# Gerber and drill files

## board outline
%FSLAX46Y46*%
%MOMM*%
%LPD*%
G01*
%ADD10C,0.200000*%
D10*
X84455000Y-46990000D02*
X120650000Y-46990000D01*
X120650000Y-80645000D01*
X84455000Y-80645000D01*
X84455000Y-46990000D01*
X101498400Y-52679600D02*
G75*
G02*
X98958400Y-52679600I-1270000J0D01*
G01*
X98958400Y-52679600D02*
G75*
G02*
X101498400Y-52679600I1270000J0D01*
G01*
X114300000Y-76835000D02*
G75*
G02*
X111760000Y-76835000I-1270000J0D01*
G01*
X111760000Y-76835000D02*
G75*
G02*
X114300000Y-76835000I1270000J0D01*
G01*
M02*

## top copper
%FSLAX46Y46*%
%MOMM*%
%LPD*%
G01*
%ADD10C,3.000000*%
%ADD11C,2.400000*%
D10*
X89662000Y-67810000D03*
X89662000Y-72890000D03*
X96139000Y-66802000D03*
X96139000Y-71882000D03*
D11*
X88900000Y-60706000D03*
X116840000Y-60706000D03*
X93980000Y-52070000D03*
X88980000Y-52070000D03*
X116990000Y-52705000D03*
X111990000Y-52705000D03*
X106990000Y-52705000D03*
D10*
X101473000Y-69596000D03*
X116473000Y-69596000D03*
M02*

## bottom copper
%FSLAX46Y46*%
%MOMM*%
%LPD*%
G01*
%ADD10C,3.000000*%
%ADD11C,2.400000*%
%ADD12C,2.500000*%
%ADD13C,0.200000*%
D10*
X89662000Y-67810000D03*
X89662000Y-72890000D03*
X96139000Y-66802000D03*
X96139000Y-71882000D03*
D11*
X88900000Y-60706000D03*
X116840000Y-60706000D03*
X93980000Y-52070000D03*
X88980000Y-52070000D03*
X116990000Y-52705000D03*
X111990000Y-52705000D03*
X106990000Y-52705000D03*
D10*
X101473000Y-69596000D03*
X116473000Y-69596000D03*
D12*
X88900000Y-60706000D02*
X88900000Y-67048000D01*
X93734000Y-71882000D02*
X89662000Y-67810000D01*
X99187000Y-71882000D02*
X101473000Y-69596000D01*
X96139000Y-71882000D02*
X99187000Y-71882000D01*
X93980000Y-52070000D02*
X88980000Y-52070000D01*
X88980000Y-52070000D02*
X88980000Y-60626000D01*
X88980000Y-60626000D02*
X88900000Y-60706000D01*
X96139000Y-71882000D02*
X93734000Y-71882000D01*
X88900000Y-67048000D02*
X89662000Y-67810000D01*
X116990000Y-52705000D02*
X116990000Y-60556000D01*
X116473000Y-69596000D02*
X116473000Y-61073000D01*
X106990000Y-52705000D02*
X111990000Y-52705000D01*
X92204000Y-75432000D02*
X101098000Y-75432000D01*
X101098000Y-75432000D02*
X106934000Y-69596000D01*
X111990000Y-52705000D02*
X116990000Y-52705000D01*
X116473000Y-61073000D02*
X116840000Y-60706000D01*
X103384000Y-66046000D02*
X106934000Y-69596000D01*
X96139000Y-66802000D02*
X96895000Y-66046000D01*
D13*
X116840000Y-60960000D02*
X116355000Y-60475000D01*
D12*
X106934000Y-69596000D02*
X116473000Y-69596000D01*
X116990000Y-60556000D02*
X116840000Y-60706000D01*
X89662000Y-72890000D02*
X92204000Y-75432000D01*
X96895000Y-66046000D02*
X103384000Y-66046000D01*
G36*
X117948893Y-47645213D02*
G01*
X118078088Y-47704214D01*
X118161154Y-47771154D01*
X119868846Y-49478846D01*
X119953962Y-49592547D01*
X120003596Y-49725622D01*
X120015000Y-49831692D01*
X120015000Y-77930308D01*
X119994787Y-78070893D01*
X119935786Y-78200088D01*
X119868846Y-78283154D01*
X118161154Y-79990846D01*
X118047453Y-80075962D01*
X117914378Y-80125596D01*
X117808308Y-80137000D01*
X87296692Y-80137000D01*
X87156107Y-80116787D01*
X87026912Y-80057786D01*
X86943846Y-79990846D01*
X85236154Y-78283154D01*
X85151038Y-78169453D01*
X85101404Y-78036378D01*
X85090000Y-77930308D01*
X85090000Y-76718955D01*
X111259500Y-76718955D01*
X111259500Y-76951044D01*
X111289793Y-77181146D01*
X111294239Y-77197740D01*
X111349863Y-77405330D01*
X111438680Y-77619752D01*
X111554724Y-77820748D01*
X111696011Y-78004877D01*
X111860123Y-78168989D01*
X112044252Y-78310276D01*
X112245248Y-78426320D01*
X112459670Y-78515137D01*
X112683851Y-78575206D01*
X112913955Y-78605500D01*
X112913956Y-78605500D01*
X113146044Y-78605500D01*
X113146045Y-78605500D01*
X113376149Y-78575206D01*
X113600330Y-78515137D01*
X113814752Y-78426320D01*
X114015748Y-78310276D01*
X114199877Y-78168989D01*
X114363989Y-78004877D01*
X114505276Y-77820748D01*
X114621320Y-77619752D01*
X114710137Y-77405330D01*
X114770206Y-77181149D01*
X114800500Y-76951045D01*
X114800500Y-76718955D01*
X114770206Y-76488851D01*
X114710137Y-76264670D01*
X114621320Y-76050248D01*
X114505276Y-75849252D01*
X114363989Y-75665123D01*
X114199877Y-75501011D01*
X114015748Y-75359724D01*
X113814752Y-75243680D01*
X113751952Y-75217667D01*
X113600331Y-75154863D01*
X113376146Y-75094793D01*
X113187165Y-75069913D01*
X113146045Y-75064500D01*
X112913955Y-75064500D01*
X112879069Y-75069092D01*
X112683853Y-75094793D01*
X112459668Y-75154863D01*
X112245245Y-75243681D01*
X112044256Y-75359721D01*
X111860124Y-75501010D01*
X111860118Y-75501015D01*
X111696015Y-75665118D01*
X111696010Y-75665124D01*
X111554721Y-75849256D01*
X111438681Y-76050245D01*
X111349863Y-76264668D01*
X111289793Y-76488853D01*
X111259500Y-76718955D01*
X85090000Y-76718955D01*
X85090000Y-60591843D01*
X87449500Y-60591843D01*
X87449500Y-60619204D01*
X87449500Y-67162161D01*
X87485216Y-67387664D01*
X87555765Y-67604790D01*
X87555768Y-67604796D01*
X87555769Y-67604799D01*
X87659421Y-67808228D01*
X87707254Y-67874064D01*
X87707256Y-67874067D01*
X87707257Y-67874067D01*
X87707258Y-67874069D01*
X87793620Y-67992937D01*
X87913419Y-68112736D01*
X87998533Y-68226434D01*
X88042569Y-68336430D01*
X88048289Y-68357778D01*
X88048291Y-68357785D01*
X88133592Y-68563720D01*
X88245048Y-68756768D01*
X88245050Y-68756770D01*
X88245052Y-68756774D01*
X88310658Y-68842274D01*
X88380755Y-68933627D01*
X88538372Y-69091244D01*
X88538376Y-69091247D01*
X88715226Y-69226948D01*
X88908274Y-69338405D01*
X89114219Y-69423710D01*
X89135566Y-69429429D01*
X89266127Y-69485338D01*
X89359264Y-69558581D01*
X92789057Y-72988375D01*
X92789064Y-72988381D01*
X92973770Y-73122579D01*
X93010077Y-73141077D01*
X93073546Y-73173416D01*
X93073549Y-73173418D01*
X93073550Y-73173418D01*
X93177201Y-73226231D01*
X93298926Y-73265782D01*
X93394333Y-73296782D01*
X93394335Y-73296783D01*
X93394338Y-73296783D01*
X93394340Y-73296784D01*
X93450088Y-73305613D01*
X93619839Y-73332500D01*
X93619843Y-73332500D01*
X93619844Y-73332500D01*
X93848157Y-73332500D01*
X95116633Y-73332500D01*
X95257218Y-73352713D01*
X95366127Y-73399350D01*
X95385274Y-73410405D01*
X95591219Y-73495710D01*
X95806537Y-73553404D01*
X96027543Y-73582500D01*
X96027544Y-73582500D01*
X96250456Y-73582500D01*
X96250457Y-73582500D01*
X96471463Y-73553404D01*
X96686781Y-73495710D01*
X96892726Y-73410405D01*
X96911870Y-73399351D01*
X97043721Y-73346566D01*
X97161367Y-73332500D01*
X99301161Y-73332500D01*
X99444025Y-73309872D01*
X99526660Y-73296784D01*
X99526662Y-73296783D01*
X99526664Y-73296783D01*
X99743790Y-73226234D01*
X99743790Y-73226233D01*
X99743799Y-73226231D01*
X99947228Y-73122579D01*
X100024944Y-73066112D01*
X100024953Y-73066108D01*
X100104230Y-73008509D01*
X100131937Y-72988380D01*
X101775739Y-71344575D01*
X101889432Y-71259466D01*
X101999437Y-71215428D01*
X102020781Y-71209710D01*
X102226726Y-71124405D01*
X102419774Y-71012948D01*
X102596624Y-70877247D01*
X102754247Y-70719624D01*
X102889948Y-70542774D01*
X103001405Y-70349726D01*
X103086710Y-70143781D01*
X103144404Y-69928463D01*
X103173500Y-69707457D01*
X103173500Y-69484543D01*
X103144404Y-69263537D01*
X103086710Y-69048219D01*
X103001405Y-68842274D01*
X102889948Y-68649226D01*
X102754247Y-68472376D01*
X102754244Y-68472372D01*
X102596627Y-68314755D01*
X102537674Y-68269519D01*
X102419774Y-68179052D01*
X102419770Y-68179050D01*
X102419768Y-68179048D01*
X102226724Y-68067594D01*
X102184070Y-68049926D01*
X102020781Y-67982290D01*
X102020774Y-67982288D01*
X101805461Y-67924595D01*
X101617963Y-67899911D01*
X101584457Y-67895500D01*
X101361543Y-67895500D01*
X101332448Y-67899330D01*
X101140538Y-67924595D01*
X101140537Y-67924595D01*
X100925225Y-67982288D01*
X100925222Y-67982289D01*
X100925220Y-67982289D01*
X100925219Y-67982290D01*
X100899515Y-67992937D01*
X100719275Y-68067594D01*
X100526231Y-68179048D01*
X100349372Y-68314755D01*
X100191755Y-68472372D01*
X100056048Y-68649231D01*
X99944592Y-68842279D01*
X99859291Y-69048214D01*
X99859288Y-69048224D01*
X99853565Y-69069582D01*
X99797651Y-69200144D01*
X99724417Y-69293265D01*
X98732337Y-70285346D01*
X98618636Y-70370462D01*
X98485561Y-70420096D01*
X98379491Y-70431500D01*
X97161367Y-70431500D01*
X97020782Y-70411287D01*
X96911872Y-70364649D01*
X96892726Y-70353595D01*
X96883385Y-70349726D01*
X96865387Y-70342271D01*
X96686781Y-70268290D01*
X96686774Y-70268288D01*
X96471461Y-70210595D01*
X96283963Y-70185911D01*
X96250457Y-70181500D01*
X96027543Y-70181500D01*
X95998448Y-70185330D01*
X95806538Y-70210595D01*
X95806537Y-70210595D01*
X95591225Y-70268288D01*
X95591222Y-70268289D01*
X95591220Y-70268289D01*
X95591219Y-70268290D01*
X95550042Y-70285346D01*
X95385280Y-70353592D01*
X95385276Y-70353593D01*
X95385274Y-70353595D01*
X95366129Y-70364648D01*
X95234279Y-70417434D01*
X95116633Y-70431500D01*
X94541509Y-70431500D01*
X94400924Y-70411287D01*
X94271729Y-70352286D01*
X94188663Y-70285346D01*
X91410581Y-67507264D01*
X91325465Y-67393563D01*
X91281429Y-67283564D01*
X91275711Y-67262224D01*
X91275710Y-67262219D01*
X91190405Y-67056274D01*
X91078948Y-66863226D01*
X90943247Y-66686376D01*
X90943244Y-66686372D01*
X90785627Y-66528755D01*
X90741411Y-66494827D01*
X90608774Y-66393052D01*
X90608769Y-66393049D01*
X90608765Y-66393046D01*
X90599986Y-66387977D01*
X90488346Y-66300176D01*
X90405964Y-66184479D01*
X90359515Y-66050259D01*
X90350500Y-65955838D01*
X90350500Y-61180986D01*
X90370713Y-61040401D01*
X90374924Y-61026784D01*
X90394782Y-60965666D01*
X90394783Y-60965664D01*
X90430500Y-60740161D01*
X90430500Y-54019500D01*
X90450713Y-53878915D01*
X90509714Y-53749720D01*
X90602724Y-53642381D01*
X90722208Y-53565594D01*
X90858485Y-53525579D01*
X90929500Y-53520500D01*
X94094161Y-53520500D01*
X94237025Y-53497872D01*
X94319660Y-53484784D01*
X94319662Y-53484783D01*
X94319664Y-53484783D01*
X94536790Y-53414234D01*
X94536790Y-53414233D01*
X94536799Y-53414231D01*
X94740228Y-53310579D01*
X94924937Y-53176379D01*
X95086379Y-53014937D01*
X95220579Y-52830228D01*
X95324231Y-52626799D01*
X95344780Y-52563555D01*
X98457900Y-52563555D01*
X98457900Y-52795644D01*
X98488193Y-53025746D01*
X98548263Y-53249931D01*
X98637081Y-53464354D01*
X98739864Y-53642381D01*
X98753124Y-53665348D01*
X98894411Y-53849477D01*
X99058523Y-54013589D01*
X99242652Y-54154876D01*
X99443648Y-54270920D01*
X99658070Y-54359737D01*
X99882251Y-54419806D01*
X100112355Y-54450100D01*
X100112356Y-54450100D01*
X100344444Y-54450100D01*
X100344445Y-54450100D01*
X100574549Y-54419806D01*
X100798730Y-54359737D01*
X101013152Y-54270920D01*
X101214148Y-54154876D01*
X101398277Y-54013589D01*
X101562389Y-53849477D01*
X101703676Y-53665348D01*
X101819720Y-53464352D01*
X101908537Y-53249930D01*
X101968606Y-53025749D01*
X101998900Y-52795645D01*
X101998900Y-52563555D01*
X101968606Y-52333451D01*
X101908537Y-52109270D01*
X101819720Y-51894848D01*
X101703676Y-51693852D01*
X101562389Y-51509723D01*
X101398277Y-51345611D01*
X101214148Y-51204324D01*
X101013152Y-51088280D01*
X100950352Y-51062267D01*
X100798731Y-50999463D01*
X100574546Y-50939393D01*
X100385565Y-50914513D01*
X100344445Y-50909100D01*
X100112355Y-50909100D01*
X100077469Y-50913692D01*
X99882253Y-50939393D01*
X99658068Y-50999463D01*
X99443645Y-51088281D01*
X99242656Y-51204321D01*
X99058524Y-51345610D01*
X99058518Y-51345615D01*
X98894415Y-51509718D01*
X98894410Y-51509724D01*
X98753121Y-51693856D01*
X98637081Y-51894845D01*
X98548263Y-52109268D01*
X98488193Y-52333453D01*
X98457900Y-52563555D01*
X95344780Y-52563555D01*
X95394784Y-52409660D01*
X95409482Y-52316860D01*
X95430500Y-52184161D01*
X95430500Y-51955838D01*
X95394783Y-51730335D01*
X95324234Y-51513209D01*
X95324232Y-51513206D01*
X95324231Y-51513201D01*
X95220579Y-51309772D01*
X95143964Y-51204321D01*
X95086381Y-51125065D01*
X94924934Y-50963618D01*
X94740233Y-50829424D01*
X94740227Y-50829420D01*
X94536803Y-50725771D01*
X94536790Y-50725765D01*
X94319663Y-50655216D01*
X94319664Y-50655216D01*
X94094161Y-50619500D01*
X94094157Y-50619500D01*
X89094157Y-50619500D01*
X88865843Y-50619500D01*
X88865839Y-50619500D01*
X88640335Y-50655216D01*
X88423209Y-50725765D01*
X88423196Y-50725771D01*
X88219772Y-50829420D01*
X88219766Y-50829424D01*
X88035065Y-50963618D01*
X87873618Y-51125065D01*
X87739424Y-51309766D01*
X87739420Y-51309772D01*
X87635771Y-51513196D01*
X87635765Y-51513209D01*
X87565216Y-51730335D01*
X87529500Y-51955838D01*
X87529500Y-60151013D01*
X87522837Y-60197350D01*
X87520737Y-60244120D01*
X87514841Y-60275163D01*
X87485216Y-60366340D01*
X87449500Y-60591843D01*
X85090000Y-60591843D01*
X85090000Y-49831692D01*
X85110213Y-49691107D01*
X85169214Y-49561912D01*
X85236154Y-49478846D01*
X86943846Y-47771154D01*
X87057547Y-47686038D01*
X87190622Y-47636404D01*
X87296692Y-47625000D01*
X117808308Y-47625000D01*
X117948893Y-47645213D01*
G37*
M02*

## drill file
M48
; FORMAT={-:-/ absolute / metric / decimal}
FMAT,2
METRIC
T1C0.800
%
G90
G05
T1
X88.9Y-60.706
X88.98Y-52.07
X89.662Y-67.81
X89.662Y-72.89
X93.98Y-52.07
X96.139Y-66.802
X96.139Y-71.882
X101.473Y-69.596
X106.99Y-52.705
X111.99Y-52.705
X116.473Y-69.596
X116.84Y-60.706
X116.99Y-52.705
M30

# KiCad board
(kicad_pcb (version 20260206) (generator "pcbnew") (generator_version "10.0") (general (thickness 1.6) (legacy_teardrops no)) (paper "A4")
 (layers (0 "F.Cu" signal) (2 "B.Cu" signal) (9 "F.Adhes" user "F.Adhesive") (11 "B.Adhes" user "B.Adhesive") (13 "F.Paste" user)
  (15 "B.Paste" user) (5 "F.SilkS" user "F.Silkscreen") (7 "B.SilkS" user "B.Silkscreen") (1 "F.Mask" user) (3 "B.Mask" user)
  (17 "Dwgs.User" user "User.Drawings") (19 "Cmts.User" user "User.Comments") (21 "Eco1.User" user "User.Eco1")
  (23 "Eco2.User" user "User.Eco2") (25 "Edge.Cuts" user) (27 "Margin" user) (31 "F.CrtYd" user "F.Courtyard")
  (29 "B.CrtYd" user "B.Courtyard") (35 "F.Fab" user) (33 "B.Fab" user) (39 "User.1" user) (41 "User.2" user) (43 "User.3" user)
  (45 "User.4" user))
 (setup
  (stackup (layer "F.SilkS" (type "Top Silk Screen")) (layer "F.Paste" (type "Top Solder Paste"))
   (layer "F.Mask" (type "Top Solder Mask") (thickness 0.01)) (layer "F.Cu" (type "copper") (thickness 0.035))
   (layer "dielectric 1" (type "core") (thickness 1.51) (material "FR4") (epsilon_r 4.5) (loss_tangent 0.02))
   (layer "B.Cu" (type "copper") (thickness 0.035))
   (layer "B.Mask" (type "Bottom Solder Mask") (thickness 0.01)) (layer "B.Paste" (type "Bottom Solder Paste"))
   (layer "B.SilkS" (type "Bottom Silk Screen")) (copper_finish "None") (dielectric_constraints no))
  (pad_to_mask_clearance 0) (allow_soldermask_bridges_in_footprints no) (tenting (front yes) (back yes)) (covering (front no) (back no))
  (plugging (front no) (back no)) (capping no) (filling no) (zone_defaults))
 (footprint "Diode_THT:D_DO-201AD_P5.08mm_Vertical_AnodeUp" (layer "F.Cu") (at 89.662 67.81 -90)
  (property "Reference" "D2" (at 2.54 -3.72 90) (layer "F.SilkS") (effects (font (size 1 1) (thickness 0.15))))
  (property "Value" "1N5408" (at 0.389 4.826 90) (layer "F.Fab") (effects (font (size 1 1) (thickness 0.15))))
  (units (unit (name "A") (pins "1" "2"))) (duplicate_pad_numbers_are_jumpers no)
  (pad "1" thru_hole circle (at 0 0 270) (size 3 3) (drill 0.8) (layers "*.Cu" "*.Mask") (remove_unused_layers no) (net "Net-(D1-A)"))
  (pad "2" thru_hole circle (at 5.08 0 270) (size 3 3) (drill 0.8) (layers "*.Cu" "*.Mask") (remove_unused_layers no) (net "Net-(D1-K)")))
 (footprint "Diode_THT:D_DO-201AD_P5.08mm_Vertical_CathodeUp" (layer "F.Cu") (at 96.139 66.802 -90)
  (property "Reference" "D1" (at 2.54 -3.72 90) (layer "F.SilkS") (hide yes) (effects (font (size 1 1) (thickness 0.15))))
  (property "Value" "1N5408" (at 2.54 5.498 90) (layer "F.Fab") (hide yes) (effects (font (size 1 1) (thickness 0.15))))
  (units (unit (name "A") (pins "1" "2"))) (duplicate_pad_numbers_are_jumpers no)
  (pad "1" thru_hole circle (at 0 0 270) (size 3 3) (drill 0.8) (layers "*.Cu" "*.Mask") (remove_unused_layers no) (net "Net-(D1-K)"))
  (pad "2" thru_hole circle (at 5.08 0 270) (size 3 3) (drill 0.8) (layers "*.Cu" "*.Mask") (remove_unused_layers no) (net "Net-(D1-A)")))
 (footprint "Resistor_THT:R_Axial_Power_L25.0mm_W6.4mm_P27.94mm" (layer "F.Cu") (at 88.9 60.706)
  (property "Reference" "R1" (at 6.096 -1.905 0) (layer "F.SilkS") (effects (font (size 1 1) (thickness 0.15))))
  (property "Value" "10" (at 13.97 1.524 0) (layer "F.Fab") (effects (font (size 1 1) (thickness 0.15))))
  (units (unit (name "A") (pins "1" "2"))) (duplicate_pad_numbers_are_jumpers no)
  (pad "1" thru_hole circle (at 0 0) (size 2.4 2.4) (drill 0.8) (layers "*.Cu" "*.Mask") (remove_unused_layers no) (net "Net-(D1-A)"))
  (pad "2" thru_hole circle (at 27.94 0) (size 2.4 2.4) (drill 0.8) (layers "*.Cu" "*.Mask") (remove_unused_layers no) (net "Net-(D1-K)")))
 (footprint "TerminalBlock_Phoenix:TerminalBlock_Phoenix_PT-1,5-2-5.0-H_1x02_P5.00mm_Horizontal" (layer "F.Cu") (at 93.98 52.07 180)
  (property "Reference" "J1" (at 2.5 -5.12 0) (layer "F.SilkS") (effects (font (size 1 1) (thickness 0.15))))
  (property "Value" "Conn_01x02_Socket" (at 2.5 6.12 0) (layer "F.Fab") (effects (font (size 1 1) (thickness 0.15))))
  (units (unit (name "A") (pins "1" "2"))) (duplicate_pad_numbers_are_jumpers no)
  (pad "1" thru_hole circle (at 0 0 180) (size 2.4 2.4) (drill 0.8) (layers "*.Cu" "*.Mask") (remove_unused_layers no) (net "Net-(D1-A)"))
  (pad "2" thru_hole circle (at 5 0 180) (size 2.4 2.4) (drill 0.8) (layers "*.Cu" "*.Mask") (remove_unused_layers no) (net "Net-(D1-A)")))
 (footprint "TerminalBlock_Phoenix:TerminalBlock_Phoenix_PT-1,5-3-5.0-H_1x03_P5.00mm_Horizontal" (layer "F.Cu") (at 116.99 52.705 180)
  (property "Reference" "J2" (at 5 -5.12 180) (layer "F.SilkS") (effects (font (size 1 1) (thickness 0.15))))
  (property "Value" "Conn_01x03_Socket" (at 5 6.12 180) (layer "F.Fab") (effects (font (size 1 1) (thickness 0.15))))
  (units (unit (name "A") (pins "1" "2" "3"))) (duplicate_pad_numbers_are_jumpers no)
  (pad "1" thru_hole circle (at 0 0 180) (size 2.4 2.4) (drill 0.8) (layers "*.Cu" "*.Mask") (remove_unused_layers no) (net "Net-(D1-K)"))
  (pad "2" thru_hole circle (at 5 0 180) (size 2.4 2.4) (drill 0.8) (layers "*.Cu" "*.Mask") (remove_unused_layers no) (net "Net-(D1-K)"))
  (pad "3" thru_hole circle (at 10 0 180) (size 2.4 2.4) (drill 0.8) (layers "*.Cu" "*.Mask") (remove_unused_layers no) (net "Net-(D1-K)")))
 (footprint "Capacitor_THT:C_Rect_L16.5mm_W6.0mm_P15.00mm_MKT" (layer "F.Cu") (at 101.473 69.596)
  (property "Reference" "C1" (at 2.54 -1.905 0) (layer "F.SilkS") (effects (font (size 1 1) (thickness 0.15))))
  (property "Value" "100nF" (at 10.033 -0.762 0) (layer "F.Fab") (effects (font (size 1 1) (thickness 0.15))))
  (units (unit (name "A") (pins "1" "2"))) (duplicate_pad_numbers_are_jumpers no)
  (pad "1" thru_hole circle (at 0 0) (size 3 3) (drill 0.8) (layers "*.Cu" "*.Mask") (remove_unused_layers no) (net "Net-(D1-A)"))
  (pad "2" thru_hole circle (at 15 0) (size 3 3) (drill 0.8) (layers "*.Cu" "*.Mask") (remove_unused_layers no) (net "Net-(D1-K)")))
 (gr_rect (start 84.455 46.99) (end 120.65 80.645) (stroke (width 0.2) (type solid)) (fill no) (layer "Edge.Cuts"))
 (gr_circle (center 100.2284 52.6796) (end 101.4984 52.6796) (stroke (width 0.2) (type solid)) (fill no) (layer "Edge.Cuts"))
 (gr_circle (center 113.03 76.835) (end 114.3 76.835) (stroke (width 0.2) (type solid)) (fill no) (layer "Edge.Cuts"))
 (segment (start 88.9 60.706) (end 88.9 67.048) (width 2.5) (layer "B.Cu") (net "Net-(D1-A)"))
 (segment (start 93.734 71.882) (end 89.662 67.81) (width 2.5) (layer "B.Cu") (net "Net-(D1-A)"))
 (segment (start 99.187 71.882) (end 101.473 69.596) (width 2.5) (layer "B.Cu") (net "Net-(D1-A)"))
 (segment (start 96.139 71.882) (end 99.187 71.882) (width 2.5) (layer "B.Cu") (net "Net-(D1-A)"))
 (segment (start 93.98 52.07) (end 88.98 52.07) (width 2.5) (layer "B.Cu") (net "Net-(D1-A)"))
 (segment (start 88.98 52.07) (end 88.98 60.626) (width 2.5) (layer "B.Cu") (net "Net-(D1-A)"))
 (segment (start 88.98 60.626) (end 88.9 60.706) (width 2.5) (layer "B.Cu") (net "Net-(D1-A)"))
 (segment (start 96.139 71.882) (end 93.734 71.882) (width 2.5) (layer "B.Cu") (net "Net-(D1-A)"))
 (segment (start 88.9 67.048) (end 89.662 67.81) (width 2.5) (layer "B.Cu") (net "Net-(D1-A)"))
 (segment (start 116.99 52.705) (end 116.99 60.556) (width 2.5) (layer "B.Cu") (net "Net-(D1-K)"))
 (segment (start 116.473 69.596) (end 116.473 61.073) (width 2.5) (layer "B.Cu") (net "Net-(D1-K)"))
 (segment (start 106.99 52.705) (end 111.99 52.705) (width 2.5) (layer "B.Cu") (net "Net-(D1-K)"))
 (segment (start 92.204 75.432) (end 101.098 75.432) (width 2.5) (layer "B.Cu") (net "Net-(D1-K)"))
 (segment (start 101.098 75.432) (end 106.934 69.596) (width 2.5) (layer "B.Cu") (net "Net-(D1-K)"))
 (segment (start 111.99 52.705) (end 116.99 52.705) (width 2.5) (layer "B.Cu") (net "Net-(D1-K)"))
 (segment (start 116.473 61.073) (end 116.84 60.706) (width 2.5) (layer "B.Cu") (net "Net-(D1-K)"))
 (segment (start 103.384 66.046) (end 106.934 69.596) (width 2.5) (layer "B.Cu") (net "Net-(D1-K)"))
 (segment (start 96.139 66.802) (end 96.895 66.046) (width 2.5) (layer "B.Cu") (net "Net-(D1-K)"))
 (segment (start 116.84 60.96) (end 116.355 60.475) (width 0.2) (layer "B.Cu") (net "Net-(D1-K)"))
 (segment (start 106.934 69.596) (end 116.473 69.596) (width 2.5) (layer "B.Cu") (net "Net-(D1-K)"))
 (segment (start 116.99 60.556) (end 116.84 60.706) (width 2.5) (layer "B.Cu") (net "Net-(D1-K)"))
 (segment (start 89.662 72.89) (end 92.204 75.432) (width 2.5) (layer "B.Cu") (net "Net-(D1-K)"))
 (segment (start 96.895 66.046) (end 103.384 66.046) (width 2.5) (layer "B.Cu") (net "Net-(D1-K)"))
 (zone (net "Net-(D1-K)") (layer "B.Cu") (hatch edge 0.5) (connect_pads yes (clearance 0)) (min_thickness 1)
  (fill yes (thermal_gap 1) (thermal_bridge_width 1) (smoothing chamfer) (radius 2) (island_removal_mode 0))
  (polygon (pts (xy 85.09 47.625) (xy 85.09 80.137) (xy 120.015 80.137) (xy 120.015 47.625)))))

